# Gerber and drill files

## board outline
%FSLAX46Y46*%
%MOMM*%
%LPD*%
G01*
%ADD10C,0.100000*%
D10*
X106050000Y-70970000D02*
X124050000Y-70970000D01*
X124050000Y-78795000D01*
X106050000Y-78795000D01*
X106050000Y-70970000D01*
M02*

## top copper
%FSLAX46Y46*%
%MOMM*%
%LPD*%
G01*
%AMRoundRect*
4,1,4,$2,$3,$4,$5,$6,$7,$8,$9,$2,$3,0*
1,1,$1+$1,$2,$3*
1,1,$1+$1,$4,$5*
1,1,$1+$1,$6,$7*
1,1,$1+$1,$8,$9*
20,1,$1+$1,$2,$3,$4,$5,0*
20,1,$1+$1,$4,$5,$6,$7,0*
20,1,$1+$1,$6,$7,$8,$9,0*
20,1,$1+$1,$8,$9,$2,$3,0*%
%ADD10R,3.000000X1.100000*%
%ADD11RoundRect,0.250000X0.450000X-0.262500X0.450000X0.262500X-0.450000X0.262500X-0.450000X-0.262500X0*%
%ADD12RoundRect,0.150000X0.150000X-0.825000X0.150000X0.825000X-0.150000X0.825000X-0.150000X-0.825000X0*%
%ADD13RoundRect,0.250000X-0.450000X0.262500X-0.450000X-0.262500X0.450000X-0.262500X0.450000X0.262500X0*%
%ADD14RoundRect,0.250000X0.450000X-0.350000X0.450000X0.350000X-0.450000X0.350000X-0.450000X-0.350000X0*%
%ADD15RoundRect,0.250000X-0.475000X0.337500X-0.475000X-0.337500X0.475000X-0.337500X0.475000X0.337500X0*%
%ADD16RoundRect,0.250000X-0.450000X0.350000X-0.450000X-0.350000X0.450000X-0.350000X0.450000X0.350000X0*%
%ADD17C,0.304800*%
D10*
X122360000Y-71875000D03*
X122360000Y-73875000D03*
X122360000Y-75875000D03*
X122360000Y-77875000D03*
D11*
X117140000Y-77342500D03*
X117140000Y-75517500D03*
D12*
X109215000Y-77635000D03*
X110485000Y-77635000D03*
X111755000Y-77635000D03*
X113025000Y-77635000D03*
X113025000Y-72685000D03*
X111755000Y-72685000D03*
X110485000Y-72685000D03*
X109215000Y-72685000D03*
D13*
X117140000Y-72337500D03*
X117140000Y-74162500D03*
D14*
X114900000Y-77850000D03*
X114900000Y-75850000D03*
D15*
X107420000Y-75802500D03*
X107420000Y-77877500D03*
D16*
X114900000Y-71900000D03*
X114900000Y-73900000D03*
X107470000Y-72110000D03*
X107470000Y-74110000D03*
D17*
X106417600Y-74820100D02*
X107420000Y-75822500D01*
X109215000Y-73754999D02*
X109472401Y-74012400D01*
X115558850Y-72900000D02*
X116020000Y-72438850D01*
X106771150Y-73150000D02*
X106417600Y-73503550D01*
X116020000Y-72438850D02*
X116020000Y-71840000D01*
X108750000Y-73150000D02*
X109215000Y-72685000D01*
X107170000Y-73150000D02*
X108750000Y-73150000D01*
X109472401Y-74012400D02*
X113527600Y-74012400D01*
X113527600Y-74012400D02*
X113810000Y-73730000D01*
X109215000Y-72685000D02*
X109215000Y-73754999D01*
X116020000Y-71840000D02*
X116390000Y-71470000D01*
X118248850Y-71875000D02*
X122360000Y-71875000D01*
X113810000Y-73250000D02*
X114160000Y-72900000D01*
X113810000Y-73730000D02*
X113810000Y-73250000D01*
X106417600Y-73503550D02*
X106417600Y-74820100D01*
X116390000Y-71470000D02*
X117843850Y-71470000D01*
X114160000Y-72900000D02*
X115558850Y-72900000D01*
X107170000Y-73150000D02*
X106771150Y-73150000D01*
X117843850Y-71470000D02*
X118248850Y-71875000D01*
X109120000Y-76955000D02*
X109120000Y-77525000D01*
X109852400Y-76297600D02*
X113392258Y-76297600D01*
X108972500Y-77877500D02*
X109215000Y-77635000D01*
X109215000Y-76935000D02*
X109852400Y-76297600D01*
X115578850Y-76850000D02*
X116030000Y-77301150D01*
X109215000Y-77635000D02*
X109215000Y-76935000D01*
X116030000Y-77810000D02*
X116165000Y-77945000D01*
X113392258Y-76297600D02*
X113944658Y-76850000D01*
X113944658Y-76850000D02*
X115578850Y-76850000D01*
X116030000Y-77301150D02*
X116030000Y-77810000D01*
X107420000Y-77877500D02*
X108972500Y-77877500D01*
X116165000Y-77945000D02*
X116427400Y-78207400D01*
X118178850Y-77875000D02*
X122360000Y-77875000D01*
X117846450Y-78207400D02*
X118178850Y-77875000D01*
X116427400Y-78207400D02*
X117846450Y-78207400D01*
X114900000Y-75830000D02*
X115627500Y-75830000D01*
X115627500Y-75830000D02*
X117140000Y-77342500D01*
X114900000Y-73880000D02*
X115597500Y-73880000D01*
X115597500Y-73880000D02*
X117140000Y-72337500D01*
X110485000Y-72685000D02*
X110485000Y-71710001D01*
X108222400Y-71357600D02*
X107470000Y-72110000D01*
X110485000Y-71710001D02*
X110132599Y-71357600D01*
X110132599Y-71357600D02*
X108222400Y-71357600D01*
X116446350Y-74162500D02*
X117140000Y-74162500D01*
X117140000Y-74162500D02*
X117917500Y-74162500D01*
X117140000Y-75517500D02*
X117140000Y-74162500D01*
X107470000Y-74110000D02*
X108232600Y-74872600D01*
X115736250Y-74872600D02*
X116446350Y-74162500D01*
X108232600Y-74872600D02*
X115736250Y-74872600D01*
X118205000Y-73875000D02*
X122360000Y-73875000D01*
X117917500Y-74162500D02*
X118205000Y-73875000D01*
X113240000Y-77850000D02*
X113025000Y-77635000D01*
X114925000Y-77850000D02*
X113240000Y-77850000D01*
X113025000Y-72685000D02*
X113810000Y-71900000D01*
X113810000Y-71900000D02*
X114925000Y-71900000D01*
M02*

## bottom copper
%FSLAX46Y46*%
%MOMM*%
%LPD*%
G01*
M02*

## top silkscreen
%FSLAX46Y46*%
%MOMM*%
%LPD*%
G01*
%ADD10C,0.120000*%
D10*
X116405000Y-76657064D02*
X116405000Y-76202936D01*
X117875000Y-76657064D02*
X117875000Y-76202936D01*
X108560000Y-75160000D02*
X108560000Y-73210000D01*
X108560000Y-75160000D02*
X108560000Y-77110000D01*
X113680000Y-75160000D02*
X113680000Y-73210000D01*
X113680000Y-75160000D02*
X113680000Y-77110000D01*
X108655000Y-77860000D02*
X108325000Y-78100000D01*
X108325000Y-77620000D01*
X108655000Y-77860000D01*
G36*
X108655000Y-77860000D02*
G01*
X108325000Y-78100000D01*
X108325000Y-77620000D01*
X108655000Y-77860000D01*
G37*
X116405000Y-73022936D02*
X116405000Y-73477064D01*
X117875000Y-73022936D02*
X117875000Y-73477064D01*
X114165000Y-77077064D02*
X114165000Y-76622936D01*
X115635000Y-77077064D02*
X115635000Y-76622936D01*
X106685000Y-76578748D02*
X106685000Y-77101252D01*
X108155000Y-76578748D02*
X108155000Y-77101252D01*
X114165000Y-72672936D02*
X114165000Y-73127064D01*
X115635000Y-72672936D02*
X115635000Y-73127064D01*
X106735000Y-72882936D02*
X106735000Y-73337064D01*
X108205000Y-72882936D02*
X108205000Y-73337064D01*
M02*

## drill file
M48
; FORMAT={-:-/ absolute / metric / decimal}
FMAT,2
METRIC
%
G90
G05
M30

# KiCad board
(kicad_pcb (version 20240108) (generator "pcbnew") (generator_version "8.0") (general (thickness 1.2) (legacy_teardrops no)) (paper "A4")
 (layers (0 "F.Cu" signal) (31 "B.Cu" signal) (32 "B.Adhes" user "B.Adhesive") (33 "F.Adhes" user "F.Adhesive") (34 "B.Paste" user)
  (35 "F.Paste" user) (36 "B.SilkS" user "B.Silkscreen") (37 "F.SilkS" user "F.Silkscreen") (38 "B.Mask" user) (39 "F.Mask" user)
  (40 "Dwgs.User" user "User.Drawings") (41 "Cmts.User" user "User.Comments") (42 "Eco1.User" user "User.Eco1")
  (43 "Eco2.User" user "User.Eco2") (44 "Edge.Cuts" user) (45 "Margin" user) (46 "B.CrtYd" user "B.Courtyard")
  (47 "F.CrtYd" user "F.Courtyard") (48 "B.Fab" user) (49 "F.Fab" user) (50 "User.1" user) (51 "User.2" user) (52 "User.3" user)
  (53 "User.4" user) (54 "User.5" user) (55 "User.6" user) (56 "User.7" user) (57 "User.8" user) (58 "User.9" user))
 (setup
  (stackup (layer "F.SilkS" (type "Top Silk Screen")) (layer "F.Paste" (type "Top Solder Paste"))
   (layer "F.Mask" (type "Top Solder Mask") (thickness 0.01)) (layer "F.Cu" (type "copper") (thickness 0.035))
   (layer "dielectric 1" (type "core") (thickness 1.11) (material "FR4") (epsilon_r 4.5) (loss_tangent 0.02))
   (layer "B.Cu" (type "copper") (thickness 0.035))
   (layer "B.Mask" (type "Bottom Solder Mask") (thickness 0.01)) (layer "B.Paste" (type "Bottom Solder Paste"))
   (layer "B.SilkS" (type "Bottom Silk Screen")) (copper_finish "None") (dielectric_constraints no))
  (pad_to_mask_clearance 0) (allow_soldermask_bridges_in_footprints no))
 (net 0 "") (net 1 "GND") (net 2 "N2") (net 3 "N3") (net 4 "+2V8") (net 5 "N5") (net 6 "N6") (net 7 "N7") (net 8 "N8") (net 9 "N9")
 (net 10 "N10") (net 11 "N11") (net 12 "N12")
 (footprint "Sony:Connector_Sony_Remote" (layer "F.Cu") (at 121.09 73.875 -90)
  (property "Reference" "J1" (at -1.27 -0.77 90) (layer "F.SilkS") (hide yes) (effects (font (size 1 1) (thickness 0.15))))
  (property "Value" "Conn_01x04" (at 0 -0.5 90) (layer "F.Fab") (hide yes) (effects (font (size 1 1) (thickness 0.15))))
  (pad "1" smd rect (at -2 -1.27 270) (size 1.1 3) (layers "F.Cu" "F.Mask") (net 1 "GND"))
  (pad "2" smd rect (at 0 -1.27 270) (size 1.1 3) (layers "F.Cu" "F.Mask") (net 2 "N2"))
  (pad "3" smd rect (at 2 -1.27 270) (size 1.1 3) (layers "F.Cu" "F.Mask") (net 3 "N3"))
  (pad "4" smd rect (at 4 -1.27 270) (size 1.1 3) (layers "F.Cu" "F.Mask") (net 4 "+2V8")))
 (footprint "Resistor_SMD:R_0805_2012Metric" (layer "F.Cu") (at 117.14 76.43 90)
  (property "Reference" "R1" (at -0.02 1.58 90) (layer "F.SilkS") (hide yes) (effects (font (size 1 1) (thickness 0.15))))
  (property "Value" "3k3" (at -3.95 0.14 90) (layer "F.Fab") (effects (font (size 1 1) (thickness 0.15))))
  (fp_line (start -0.227064 -0.735) (end 0.227064 -0.735) (stroke (width 0.12) (type solid)) (layer "F.SilkS"))
  (fp_line (start -0.227064 0.735) (end 0.227064 0.735) (stroke (width 0.12) (type solid)) (layer "F.SilkS"))
  (pad "1" smd roundrect (at -0.9125 0 90) (size 1.025 1.4) (layers "F.Cu" "F.Paste" "F.Mask") (roundrect_rratio 0.243902) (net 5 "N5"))
  (pad "2" smd roundrect (at 0.9125 0 90) (size 1.025 1.4) (layers "F.Cu" "F.Paste" "F.Mask") (roundrect_rratio 0.243902) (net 2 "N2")))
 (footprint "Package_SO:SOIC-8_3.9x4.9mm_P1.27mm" (layer "F.Cu") (at 111.12 75.16 90)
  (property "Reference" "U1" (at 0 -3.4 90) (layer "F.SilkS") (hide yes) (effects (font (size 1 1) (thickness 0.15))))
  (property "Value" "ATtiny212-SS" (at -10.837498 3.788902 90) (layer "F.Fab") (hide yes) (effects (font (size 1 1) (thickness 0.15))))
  (fp_line (start 0 -2.56) (end 1.95 -2.56) (stroke (width 0.12) (type solid)) (layer "F.SilkS"))
  (fp_line (start 0 -2.56) (end -1.95 -2.56) (stroke (width 0.12) (type solid)) (layer "F.SilkS"))
  (fp_line (start 0 2.56) (end 1.95 2.56) (stroke (width 0.12) (type solid)) (layer "F.SilkS"))
  (fp_line (start 0 2.56) (end -1.95 2.56) (stroke (width 0.12) (type solid)) (layer "F.SilkS"))
  (fp_poly
   (pts (xy -2.7 -2.465) (xy -2.94 -2.795) (xy -2.46 -2.795) (xy -2.7 -2.465)) (stroke (width 0.12) (type solid)) (fill solid)
   (layer "F.SilkS"))
  (pad "1" smd roundrect (at -2.475 -1.905 90) (size 1.95 0.6) (layers "F.Cu" "F.Paste" "F.Mask") (roundrect_rratio 0.25) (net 4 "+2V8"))
  (pad "2" smd roundrect (at -2.475 -0.635 90) (size 1.95 0.6) (layers "F.Cu" "F.Paste" "F.Mask") (roundrect_rratio 0.25) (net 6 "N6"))
  (pad "3" smd roundrect (at -2.475 0.635 90) (size 1.95 0.6) (layers "F.Cu" "F.Paste" "F.Mask") (roundrect_rratio 0.25) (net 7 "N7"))
  (pad "4" smd roundrect (at -2.475 1.905 90) (size 1.95 0.6) (layers "F.Cu" "F.Paste" "F.Mask") (roundrect_rratio 0.25) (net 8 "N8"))
  (pad "5" smd roundrect (at 2.475 1.905 90) (size 1.95 0.6) (layers "F.Cu" "F.Paste" "F.Mask") (roundrect_rratio 0.25) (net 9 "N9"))
  (pad "6" smd roundrect (at 2.475 0.635 90) (size 1.95 0.6) (layers "F.Cu" "F.Paste" "F.Mask") (roundrect_rratio 0.25) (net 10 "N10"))
  (pad "7" smd roundrect (at 2.475 -0.635 90) (size 1.95 0.6) (layers "F.Cu" "F.Paste" "F.Mask") (roundrect_rratio 0.25) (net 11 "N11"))
  (pad "8" smd roundrect (at 2.475 -1.905 90) (size 1.95 0.6) (layers "F.Cu" "F.Paste" "F.Mask") (roundrect_rratio 0.25) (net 1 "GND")))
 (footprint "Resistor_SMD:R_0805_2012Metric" (layer "F.Cu") (at 117.14 73.25 -90)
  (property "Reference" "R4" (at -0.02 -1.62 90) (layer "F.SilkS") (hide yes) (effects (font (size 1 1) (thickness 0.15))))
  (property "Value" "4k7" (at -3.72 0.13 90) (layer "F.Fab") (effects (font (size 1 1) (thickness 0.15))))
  (fp_line (start -0.227064 0.735) (end 0.227064 0.735) (stroke (width 0.12) (type solid)) (layer "F.SilkS"))
  (fp_line (start -0.227064 -0.735) (end 0.227064 -0.735) (stroke (width 0.12) (type solid)) (layer "F.SilkS"))
  (pad "1" smd roundrect (at -0.9125 0 270) (size 1.025 1.4) (layers "F.Cu" "F.Paste" "F.Mask") (roundrect_rratio 0.243902) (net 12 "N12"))
  (pad "2" smd roundrect (at 0.9125 0 270) (size 1.025 1.4) (layers "F.Cu" "F.Paste" "F.Mask") (roundrect_rratio 0.243902) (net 2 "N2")))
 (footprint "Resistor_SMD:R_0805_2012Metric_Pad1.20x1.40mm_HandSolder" (layer "F.Cu") (at 114.9 76.85 90)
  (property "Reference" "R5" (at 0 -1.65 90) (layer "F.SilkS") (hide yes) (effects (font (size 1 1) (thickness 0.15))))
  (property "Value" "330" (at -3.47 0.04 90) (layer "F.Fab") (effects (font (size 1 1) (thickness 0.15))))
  (fp_line (start -0.227064 -0.735) (end 0.227064 -0.735) (stroke (width 0.12) (type solid)) (layer "F.SilkS"))
  (fp_line (start -0.227064 0.735) (end 0.227064 0.735) (stroke (width 0.12) (type solid)) (layer "F.SilkS"))
  (pad "1" smd roundrect (at -1 0 90) (size 1.2 1.4) (layers "F.Cu" "F.Paste" "F.Mask") (roundrect_rratio 0.208333) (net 8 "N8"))
  (pad "2" smd roundrect (at 1 0 90) (size 1.2 1.4) (layers "F.Cu" "F.Paste" "F.Mask") (roundrect_rratio 0.208333) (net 5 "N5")))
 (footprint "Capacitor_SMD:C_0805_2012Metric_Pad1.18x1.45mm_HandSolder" (layer "F.Cu") (at 107.42 76.84 -90)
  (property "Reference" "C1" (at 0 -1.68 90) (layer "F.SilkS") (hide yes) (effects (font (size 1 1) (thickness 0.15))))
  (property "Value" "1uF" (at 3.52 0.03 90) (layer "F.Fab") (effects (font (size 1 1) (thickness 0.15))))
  (fp_line (start -0.261252 0.735) (end 0.261252 0.735) (stroke (width 0.12) (type solid)) (layer "F.SilkS"))
  (fp_line (start -0.261252 -0.735) (end 0.261252 -0.735) (stroke (width 0.12) (type solid)) (layer "F.SilkS"))
  (pad "1" smd roundrect (at -1.0375 0 270) (size 1.175 1.45) (layers "F.Cu" "F.Paste" "F.Mask") (roundrect_rratio 0.212766) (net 1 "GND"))
  (pad "2" smd roundrect (at 1.0375 0 270) (size 1.175 1.45) (layers "F.Cu" "F.Paste" "F.Mask") (roundrect_rratio 0.212766) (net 4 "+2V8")))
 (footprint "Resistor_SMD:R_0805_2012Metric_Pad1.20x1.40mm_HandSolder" (layer "F.Cu") (at 114.9 72.9 -90)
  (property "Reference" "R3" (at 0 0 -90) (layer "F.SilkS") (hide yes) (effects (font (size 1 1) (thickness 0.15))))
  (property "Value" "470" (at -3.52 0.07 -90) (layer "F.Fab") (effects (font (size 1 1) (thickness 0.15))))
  (fp_line (start -0.227064 0.735) (end 0.227064 0.735) (stroke (width 0.12) (type solid)) (layer "F.SilkS"))
  (fp_line (start -0.227064 -0.735) (end 0.227064 -0.735) (stroke (width 0.12) (type solid)) (layer "F.SilkS"))
  (pad "1" smd roundrect (at -1 0 270) (size 1.2 1.4) (layers "F.Cu" "F.Paste" "F.Mask") (roundrect_rratio 0.208333) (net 9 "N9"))
  (pad "2" smd roundrect (at 1 0 270) (size 1.2 1.4) (layers "F.Cu" "F.Paste" "F.Mask") (roundrect_rratio 0.208333) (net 12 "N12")))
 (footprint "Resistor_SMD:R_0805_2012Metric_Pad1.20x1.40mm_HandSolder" (layer "F.Cu") (at 107.47 73.11 -90)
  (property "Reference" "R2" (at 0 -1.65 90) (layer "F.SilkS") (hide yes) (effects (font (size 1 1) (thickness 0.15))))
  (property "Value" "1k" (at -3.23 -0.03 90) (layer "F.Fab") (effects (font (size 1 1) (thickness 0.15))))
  (fp_line (start -0.227064 0.735) (end 0.227064 0.735) (stroke (width 0.12) (type solid)) (layer "F.SilkS"))
  (fp_line (start -0.227064 -0.735) (end 0.227064 -0.735) (stroke (width 0.12) (type solid)) (layer "F.SilkS"))
  (pad "1" smd roundrect (at -1 0 270) (size 1.2 1.4) (layers "F.Cu" "F.Paste" "F.Mask") (roundrect_rratio 0.208333) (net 11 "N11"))
  (pad "2" smd roundrect (at 1 0 270) (size 1.2 1.4) (layers "F.Cu" "F.Paste" "F.Mask") (roundrect_rratio 0.208333) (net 2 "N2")))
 (gr_rect (start 106.05 70.97) (end 124.05 78.795) (stroke (width 0.1) (type default)) (fill none) (layer "Edge.Cuts"))
 (segment (start 106.4176 74.8201) (end 107.42 75.8225) (width 0.3048) (layer "F.Cu") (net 1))
 (segment (start 109.215 73.754999) (end 109.472401 74.0124) (width 0.3048) (layer "F.Cu") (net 1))
 (segment (start 115.55885 72.9) (end 116.02 72.43885) (width 0.3048) (layer "F.Cu") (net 1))
 (segment (start 106.77115 73.15) (end 106.4176 73.50355) (width 0.3048) (layer "F.Cu") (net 1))
 (segment (start 116.02 72.43885) (end 116.02 71.84) (width 0.3048) (layer "F.Cu") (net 1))
 (segment (start 108.75 73.15) (end 109.215 72.685) (width 0.3048) (layer "F.Cu") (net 1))
 (segment (start 107.17 73.15) (end 108.75 73.15) (width 0.3048) (layer "F.Cu") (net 1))
 (segment (start 109.472401 74.0124) (end 113.5276 74.0124) (width 0.3048) (layer "F.Cu") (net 1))
 (segment (start 113.5276 74.0124) (end 113.81 73.73) (width 0.3048) (layer "F.Cu") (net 1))
 (segment (start 109.215 72.685) (end 109.215 73.754999) (width 0.3048) (layer "F.Cu") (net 1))
 (segment (start 116.02 71.84) (end 116.39 71.47) (width 0.3048) (layer "F.Cu") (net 1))
 (segment (start 118.24885 71.875) (end 122.36 71.875) (width 0.3048) (layer "F.Cu") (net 1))
 (segment (start 113.81 73.25) (end 114.16 72.9) (width 0.3048) (layer "F.Cu") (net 1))
 (segment (start 113.81 73.73) (end 113.81 73.25) (width 0.3048) (layer "F.Cu") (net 1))
 (segment (start 106.4176 73.50355) (end 106.4176 74.8201) (width 0.3048) (layer "F.Cu") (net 1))
 (segment (start 116.39 71.47) (end 117.84385 71.47) (width 0.3048) (layer "F.Cu") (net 1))
 (segment (start 114.16 72.9) (end 115.55885 72.9) (width 0.3048) (layer "F.Cu") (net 1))
 (segment (start 107.17 73.15) (end 106.77115 73.15) (width 0.3048) (layer "F.Cu") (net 1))
 (segment (start 117.84385 71.47) (end 118.24885 71.875) (width 0.3048) (layer "F.Cu") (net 1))
 (segment (start 109.12 76.955) (end 109.12 77.525) (width 0.3048) (layer "F.Cu") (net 4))
 (segment (start 109.8524 76.2976) (end 113.392258 76.2976) (width 0.3048) (layer "F.Cu") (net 4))
 (segment (start 108.9725 77.8775) (end 109.215 77.635) (width 0.3048) (layer "F.Cu") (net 4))
 (segment (start 109.215 76.935) (end 109.8524 76.2976) (width 0.3048) (layer "F.Cu") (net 4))
 (segment (start 115.57885 76.85) (end 116.03 77.30115) (width 0.3048) (layer "F.Cu") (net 4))
 (segment (start 109.215 77.635) (end 109.215 76.935) (width 0.3048) (layer "F.Cu") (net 4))
 (segment (start 116.03 77.81) (end 116.165 77.945) (width 0.3048) (layer "F.Cu") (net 4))
 (segment (start 113.392258 76.2976) (end 113.944658 76.85) (width 0.3048) (layer "F.Cu") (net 4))
 (segment (start 113.944658 76.85) (end 115.57885 76.85) (width 0.3048) (layer "F.Cu") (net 4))
 (segment (start 116.03 77.30115) (end 116.03 77.81) (width 0.3048) (layer "F.Cu") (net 4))
 (segment (start 107.42 77.8775) (end 108.9725 77.8775) (width 0.3048) (layer "F.Cu") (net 4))
 (segment (start 116.165 77.945) (end 116.4274 78.2074) (width 0.3048) (layer "F.Cu") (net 4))
 (segment (start 118.17885 77.875) (end 122.36 77.875) (width 0.3048) (layer "F.Cu") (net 4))
 (segment (start 117.84645 78.2074) (end 118.17885 77.875) (width 0.3048) (layer "F.Cu") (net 4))
 (segment (start 116.4274 78.2074) (end 117.84645 78.2074) (width 0.3048) (layer "F.Cu") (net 4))
 (segment (start 114.9 75.83) (end 115.6275 75.83) (width 0.3048) (layer "F.Cu") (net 5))
 (segment (start 115.6275 75.83) (end 117.14 77.3425) (width 0.3048) (layer "F.Cu") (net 5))
 (segment (start 114.9 73.88) (end 115.5975 73.88) (width 0.3048) (layer "F.Cu") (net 12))
 (segment (start 115.5975 73.88) (end 117.14 72.3375) (width 0.3048) (layer "F.Cu") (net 12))
 (segment (start 110.485 72.685) (end 110.485 71.710001) (width 0.3048) (layer "F.Cu") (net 11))
 (segment (start 108.2224 71.3576) (end 107.47 72.11) (width 0.3048) (layer "F.Cu") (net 11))
 (segment (start 110.485 71.710001) (end 110.132599 71.3576) (width 0.3048) (layer "F.Cu") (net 11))
 (segment (start 110.132599 71.3576) (end 108.2224 71.3576) (width 0.3048) (layer "F.Cu") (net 11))
 (segment (start 116.44635 74.1625) (end 117.14 74.1625) (width 0.3048) (layer "F.Cu") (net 2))
 (segment (start 117.14 74.1625) (end 117.9175 74.1625) (width 0.3048) (layer "F.Cu") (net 2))
 (segment (start 117.14 75.5175) (end 117.14 74.1625) (width 0.3048) (layer "F.Cu") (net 2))
 (segment (start 107.47 74.11) (end 108.2326 74.8726) (width 0.3048) (layer "F.Cu") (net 2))
 (segment (start 115.73625 74.8726) (end 116.44635 74.1625) (width 0.3048) (layer "F.Cu") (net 2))
 (segment (start 108.2326 74.8726) (end 115.73625 74.8726) (width 0.3048) (layer "F.Cu") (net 2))
 (segment (start 118.205 73.875) (end 122.36 73.875) (width 0.3048) (layer "F.Cu") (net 2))
 (segment (start 117.9175 74.1625) (end 118.205 73.875) (width 0.3048) (layer "F.Cu") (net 2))
 (segment (start 113.24 77.85) (end 113.025 77.635) (width 0.3048) (layer "F.Cu") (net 8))
 (segment (start 114.925 77.85) (end 113.24 77.85) (width 0.3048) (layer "F.Cu") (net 8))
 (segment (start 113.025 72.685) (end 113.81 71.9) (width 0.3048) (layer "F.Cu") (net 9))
 (segment (start 113.81 71.9) (end 114.925 71.9) (width 0.3048) (layer "F.Cu") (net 9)))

